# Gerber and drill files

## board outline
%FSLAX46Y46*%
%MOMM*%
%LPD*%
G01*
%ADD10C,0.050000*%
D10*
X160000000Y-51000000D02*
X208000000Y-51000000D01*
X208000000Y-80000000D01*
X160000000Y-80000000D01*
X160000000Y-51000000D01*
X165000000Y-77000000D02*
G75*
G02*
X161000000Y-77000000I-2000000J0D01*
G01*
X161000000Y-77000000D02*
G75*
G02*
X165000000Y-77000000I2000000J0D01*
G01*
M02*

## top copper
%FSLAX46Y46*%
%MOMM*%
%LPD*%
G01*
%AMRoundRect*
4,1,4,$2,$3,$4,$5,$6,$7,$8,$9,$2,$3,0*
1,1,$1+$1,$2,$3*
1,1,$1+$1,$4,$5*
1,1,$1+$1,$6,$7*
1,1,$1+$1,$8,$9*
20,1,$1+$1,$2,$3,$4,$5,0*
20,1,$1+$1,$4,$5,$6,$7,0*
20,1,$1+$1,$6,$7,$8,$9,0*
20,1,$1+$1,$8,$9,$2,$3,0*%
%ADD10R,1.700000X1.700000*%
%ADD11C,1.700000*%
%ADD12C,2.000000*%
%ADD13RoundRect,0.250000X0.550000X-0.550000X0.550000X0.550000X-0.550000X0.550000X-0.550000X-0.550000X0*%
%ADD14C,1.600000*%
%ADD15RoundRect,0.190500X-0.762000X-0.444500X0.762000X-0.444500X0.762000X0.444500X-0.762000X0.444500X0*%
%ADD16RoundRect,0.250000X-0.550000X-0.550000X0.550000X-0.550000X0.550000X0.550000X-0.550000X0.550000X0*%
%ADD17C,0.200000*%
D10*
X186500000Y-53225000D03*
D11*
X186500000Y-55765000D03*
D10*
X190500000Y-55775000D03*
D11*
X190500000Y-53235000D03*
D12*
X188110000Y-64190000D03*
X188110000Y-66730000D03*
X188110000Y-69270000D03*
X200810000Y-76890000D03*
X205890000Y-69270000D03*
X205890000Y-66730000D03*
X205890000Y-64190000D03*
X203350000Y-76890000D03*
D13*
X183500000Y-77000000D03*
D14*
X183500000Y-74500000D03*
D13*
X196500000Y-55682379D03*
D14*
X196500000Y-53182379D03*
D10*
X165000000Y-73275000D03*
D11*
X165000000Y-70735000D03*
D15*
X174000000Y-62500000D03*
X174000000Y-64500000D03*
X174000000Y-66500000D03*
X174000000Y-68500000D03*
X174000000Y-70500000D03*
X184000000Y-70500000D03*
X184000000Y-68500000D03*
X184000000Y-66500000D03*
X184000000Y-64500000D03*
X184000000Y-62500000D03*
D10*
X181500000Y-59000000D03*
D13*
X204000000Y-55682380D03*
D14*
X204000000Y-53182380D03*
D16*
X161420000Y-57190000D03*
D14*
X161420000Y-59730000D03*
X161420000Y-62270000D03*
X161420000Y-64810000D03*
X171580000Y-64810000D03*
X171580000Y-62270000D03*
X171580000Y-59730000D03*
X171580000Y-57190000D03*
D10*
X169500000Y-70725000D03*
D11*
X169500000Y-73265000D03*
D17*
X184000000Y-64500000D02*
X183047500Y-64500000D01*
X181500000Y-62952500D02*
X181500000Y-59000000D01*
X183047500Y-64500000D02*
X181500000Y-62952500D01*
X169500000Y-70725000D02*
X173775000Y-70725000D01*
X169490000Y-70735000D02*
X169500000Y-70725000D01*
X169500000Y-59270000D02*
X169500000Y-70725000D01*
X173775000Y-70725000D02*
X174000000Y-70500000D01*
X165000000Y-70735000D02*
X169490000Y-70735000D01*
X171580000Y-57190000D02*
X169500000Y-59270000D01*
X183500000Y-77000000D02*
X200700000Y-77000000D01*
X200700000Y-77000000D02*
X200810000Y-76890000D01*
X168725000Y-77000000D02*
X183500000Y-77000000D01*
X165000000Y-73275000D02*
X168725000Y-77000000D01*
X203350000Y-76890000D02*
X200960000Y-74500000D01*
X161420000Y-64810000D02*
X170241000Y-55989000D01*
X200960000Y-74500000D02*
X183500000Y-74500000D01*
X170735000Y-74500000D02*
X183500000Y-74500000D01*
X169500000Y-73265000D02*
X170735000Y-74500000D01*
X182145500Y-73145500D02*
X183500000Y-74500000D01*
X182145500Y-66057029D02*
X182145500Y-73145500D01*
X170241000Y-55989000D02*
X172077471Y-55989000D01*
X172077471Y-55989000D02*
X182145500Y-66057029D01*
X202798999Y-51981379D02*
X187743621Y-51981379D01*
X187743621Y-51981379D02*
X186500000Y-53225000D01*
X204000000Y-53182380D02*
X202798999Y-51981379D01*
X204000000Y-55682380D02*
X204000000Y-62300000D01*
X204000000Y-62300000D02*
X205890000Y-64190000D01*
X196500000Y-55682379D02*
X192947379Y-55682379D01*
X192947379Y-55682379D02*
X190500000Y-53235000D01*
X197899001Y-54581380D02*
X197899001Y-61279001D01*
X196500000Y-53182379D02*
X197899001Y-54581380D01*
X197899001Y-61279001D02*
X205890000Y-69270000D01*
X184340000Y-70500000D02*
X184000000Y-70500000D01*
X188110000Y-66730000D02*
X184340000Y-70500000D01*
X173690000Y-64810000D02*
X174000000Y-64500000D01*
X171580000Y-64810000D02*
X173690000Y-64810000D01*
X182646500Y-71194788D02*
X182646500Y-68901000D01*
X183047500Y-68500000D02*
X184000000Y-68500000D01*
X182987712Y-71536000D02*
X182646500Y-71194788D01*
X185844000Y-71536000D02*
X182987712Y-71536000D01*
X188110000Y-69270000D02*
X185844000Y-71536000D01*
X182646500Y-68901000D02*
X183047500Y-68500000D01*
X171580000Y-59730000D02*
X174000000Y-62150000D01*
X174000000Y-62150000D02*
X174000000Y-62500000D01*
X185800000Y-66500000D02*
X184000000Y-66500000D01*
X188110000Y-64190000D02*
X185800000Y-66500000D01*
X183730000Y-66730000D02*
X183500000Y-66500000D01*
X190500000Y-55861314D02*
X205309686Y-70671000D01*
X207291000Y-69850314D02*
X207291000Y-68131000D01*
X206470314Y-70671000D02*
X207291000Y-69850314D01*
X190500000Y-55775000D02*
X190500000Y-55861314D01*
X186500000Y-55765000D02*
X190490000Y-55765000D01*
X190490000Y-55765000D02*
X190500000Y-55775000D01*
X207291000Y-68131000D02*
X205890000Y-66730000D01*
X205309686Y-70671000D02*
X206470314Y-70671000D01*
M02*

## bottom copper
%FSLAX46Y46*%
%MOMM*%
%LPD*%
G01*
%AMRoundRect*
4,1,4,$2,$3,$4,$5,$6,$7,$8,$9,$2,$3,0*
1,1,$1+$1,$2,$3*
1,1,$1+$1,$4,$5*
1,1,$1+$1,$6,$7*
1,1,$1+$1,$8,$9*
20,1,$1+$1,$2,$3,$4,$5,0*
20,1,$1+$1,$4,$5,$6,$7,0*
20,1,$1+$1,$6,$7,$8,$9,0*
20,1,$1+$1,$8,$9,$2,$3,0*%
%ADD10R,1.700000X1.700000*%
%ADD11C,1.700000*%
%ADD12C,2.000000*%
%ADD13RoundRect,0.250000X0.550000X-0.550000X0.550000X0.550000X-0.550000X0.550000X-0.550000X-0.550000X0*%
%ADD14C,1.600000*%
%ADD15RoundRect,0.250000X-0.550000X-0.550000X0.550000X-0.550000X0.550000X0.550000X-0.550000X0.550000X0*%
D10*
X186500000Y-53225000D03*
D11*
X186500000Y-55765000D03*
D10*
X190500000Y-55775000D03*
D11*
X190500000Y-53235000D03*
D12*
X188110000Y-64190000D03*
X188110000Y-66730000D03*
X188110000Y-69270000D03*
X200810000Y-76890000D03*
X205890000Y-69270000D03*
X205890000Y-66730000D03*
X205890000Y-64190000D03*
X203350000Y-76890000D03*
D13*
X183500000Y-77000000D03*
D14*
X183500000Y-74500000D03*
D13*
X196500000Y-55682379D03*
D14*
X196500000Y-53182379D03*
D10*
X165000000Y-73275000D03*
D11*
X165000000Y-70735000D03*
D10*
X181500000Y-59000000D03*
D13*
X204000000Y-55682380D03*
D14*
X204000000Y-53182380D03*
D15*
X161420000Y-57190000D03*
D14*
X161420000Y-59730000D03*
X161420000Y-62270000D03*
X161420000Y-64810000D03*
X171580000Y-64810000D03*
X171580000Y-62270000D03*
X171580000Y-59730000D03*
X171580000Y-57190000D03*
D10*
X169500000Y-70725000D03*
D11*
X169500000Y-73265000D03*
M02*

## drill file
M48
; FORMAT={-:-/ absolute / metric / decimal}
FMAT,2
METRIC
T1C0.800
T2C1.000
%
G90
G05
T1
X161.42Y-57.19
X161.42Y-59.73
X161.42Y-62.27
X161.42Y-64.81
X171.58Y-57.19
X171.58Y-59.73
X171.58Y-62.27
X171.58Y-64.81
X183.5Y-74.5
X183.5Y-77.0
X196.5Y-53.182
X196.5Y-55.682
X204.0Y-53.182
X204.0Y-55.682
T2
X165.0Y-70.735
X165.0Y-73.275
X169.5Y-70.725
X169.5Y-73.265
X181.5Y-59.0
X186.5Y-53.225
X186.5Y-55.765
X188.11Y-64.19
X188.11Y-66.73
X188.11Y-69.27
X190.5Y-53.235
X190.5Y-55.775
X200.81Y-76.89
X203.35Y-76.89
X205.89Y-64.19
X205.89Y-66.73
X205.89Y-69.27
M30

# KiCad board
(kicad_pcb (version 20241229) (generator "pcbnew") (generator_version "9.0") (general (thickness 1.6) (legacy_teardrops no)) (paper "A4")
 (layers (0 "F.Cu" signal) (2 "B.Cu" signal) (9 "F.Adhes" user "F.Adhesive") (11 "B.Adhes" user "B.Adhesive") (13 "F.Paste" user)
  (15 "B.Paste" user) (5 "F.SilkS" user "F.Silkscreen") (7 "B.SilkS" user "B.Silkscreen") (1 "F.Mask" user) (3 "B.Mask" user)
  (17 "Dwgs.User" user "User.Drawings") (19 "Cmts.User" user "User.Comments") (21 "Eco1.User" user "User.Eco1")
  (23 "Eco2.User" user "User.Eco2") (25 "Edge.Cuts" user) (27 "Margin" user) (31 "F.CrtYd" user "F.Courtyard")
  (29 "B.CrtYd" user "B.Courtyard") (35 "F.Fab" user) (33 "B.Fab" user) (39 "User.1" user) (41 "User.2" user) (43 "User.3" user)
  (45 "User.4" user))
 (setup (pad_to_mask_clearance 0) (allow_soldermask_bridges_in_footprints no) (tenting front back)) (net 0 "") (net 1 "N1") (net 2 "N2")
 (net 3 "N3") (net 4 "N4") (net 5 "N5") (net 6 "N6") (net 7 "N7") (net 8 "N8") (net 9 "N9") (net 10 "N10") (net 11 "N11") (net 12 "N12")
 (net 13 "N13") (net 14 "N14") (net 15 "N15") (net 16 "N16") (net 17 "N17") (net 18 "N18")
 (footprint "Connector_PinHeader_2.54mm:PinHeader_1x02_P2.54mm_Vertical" (layer "F.Cu") (at 186.5 53.225)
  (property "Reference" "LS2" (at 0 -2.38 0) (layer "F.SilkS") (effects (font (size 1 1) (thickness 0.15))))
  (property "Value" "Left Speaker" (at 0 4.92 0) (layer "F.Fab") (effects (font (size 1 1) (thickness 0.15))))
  (pad "1" thru_hole rect (at 0 0) (size 1.7 1.7) (drill 1) (layers "*.Cu" "*.Mask") (remove_unused_layers no) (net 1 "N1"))
  (pad "2" thru_hole circle (at 0 2.54) (size 1.7 1.7) (drill 1) (layers "*.Cu" "*.Mask") (remove_unused_layers no) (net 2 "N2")))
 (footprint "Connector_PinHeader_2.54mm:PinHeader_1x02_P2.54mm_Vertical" (layer "F.Cu") (at 190.5 55.775 180)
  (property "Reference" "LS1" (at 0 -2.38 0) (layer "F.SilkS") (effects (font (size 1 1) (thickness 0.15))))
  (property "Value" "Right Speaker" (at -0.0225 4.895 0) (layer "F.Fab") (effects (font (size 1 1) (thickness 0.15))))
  (pad "1" thru_hole rect (at 0 0 180) (size 1.7 1.7) (drill 1) (layers "*.Cu" "*.Mask") (remove_unused_layers no) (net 2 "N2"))
  (pad "2" thru_hole circle (at 0 2.54 180) (size 1.7 1.7) (drill 1) (layers "*.Cu" "*.Mask") (remove_unused_layers no) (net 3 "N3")))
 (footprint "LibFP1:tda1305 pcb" (layer "F.Cu") (at 198.27 66.73)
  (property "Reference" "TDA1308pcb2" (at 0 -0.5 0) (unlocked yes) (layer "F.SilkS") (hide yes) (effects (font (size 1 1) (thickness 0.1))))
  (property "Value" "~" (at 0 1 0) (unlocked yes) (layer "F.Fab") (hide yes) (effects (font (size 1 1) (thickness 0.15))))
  (pad "1" thru_hole circle (at -10.16 -2.54) (size 2 2) (drill 1) (layers "*.Cu" "*.Mask") (remove_unused_layers no) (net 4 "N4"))
  (pad "2" thru_hole circle (at -10.16 0) (size 2 2) (drill 1) (layers "*.Cu" "*.Mask") (remove_unused_layers no) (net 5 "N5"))
  (pad "3" thru_hole circle (at -10.16 2.54) (size 2 2) (drill 1) (layers "*.Cu" "*.Mask") (remove_unused_layers no) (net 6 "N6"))
  (pad "4" thru_hole circle (at 2.54 10.16) (size 2 2) (drill 1) (layers "*.Cu" "*.Mask") (remove_unused_layers no) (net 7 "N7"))
  (pad "5" thru_hole circle (at 7.62 2.54) (size 2 2) (drill 1) (layers "*.Cu" "*.Mask") (remove_unused_layers no) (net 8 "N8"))
  (pad "6" thru_hole circle (at 7.62 0) (size 2 2) (drill 1) (layers "*.Cu" "*.Mask") (remove_unused_layers no) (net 2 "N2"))
  (pad "7" thru_hole circle (at 7.62 -2.54) (size 2 2) (drill 1) (layers "*.Cu" "*.Mask") (remove_unused_layers no) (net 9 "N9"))
  (pad "8" thru_hole circle (at 5.08 10.16) (size 2 2) (drill 1) (layers "*.Cu" "*.Mask") (remove_unused_layers no) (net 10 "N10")))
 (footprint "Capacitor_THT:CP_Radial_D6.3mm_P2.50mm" (layer "F.Cu") (at 183.5 77 90)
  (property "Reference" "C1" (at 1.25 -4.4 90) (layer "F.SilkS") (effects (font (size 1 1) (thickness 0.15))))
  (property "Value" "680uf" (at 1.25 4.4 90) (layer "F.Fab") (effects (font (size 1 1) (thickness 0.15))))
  (pad "1" thru_hole roundrect (at 0 0 90) (size 1.6 1.6) (drill 0.8) (layers "*.Cu" "*.Mask") (remove_unused_layers no)
   (roundrect_rratio 0.15625) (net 7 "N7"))
  (pad "2" thru_hole circle (at 2.5 0 90) (size 1.6 1.6) (drill 0.8) (layers "*.Cu" "*.Mask") (remove_unused_layers no) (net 10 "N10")))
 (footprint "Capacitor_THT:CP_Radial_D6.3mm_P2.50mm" (layer "F.Cu") (at 196.5 55.682379 90)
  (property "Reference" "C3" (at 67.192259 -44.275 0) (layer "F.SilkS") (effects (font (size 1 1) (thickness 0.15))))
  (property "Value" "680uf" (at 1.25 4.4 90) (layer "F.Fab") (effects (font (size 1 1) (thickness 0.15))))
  (pad "1" thru_hole roundrect (at 0 0 90) (size 1.6 1.6) (drill 0.8) (layers "*.Cu" "*.Mask") (remove_unused_layers no)
   (roundrect_rratio 0.15625) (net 3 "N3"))
  (pad "2" thru_hole circle (at 2.5 0 90) (size 1.6 1.6) (drill 0.8) (layers "*.Cu" "*.Mask") (remove_unused_layers no) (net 8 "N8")))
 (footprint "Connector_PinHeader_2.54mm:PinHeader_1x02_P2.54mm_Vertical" (layer "F.Cu") (at 165 73.275 180)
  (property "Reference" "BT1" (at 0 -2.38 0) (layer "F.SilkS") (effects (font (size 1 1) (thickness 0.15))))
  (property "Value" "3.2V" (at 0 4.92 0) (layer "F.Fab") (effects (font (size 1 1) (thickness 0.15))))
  (pad "1" thru_hole rect (at 0 0 180) (size 1.7 1.7) (drill 1) (layers "*.Cu" "*.Mask") (remove_unused_layers no) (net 7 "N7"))
  (pad "2" thru_hole circle (at 0 2.54 180) (size 1.7 1.7) (drill 1) (layers "*.Cu" "*.Mask") (remove_unused_layers no) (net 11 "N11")))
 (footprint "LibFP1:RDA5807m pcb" (layer "F.Cu") (at 179 66.5)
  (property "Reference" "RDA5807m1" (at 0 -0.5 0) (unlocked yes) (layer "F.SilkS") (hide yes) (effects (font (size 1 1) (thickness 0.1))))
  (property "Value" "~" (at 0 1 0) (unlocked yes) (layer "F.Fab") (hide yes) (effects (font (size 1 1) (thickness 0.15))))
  (pad "1" smd roundrect (at -5 -4) (size 1.905 1.27) (layers "F.Cu" "F.Mask" "F.Paste") (roundrect_rratio 0.15) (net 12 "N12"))
  (pad "2" smd roundrect (at -5 -2) (size 1.905 1.27) (layers "F.Cu" "F.Mask" "F.Paste") (roundrect_rratio 0.15) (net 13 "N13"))
  (pad "3" smd roundrect (at -5 0) (size 1.905 1.27) (layers "F.Cu" "F.Mask" "F.Paste") (roundrect_rratio 0.15))
  (pad "4" smd roundrect (at -5 2) (size 1.905 1.27) (layers "F.Cu" "F.Mask" "F.Paste") (roundrect_rratio 0.15))
  (pad "5" smd roundrect (at -5 4) (size 1.905 1.27) (layers "F.Cu" "F.Mask" "F.Paste") (roundrect_rratio 0.15) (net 11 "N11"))
  (pad "6" smd roundrect (at 5 4) (size 1.905 1.27) (layers "F.Cu" "F.Mask" "F.Paste") (roundrect_rratio 0.15) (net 5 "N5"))
  (pad "7" smd roundrect (at 5 2) (size 1.905 1.27) (layers "F.Cu" "F.Mask" "F.Paste") (roundrect_rratio 0.15) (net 6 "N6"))
  (pad "8" smd roundrect (at 5 0) (size 1.905 1.27) (layers "F.Cu" "F.Mask" "F.Paste") (roundrect_rratio 0.15) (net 4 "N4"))
  (pad "9" smd roundrect (at 5 -2) (size 1.905 1.27) (layers "F.Cu" "F.Mask" "F.Paste") (roundrect_rratio 0.15) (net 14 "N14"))
  (pad "10" smd roundrect (at 5 -4) (size 1.905 1.27) (layers "F.Cu" "F.Mask" "F.Paste") (roundrect_rratio 0.15)))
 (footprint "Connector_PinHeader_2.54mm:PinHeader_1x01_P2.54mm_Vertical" (layer "F.Cu") (at 181.5 59)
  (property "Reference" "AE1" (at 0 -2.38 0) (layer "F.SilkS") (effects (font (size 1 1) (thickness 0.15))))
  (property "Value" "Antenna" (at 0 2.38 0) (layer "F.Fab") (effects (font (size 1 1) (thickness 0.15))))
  (pad "1" thru_hole rect (at 0 0) (size 1.7 1.7) (drill 1) (layers "*.Cu" "*.Mask") (remove_unused_layers no) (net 14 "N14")))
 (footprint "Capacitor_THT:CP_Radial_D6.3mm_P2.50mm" (layer "F.Cu") (at 204 55.68238 90)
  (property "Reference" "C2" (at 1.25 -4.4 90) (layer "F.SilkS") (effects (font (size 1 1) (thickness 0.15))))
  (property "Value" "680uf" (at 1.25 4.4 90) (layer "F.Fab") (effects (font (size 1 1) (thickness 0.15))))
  (pad "1" thru_hole roundrect (at 0 0 90) (size 1.6 1.6) (drill 0.8) (layers "*.Cu" "*.Mask") (remove_unused_layers no)
   (roundrect_rratio 0.15625) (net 9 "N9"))
  (pad "2" thru_hole circle (at 2.5 0 90) (size 1.6 1.6) (drill 0.8) (layers "*.Cu" "*.Mask") (remove_unused_layers no) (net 1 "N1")))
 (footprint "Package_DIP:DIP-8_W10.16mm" (layer "F.Cu") (at 161.42 57.19)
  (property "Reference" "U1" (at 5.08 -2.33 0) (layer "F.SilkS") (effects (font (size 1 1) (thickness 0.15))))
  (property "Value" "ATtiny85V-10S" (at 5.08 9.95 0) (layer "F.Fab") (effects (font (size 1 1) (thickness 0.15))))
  (pad "1" thru_hole roundrect (at 0 0) (size 1.6 1.6) (drill 0.8) (layers "*.Cu" "*.Mask") (remove_unused_layers no)
   (roundrect_rratio 0.15625) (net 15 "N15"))
  (pad "2" thru_hole circle (at 0 2.54) (size 1.6 1.6) (drill 0.8) (layers "*.Cu" "*.Mask") (remove_unused_layers no) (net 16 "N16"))
  (pad "3" thru_hole circle (at 0 5.08) (size 1.6 1.6) (drill 0.8) (layers "*.Cu" "*.Mask") (remove_unused_layers no) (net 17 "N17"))
  (pad "4" thru_hole circle (at 0 7.62) (size 1.6 1.6) (drill 0.8) (layers "*.Cu" "*.Mask") (remove_unused_layers no) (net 10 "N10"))
  (pad "5" thru_hole circle (at 10.16 7.62) (size 1.6 1.6) (drill 0.8) (layers "*.Cu" "*.Mask") (remove_unused_layers no) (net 13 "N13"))
  (pad "6" thru_hole circle (at 10.16 5.08) (size 1.6 1.6) (drill 0.8) (layers "*.Cu" "*.Mask") (remove_unused_layers no) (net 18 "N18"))
  (pad "7" thru_hole circle (at 10.16 2.54) (size 1.6 1.6) (drill 0.8) (layers "*.Cu" "*.Mask") (remove_unused_layers no) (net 12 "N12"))
  (pad "8" thru_hole circle (at 10.16 0) (size 1.6 1.6) (drill 0.8) (layers "*.Cu" "*.Mask") (remove_unused_layers no) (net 11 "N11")))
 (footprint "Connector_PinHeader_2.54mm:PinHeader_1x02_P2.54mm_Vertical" (layer "F.Cu") (at 169.5 70.725)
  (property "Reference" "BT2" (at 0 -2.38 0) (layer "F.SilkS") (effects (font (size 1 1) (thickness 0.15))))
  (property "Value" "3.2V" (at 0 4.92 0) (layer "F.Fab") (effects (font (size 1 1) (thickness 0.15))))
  (pad "1" thru_hole rect (at 0 0) (size 1.7 1.7) (drill 1) (layers "*.Cu" "*.Mask") (remove_unused_layers no) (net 11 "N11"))
  (pad "2" thru_hole circle (at 0 2.54) (size 1.7 1.7) (drill 1) (layers "*.Cu" "*.Mask") (remove_unused_layers no) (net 10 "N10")))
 (gr_rect (start 160 51) (end 208 80) (stroke (width 0.05) (type default)) (fill no) (layer "Edge.Cuts"))
 (gr_circle (center 163 77) (end 163 79) (stroke (width 0.05) (type default)) (fill no) (layer "Edge.Cuts"))
 (segment (start 184 64.5) (end 183.0475 64.5) (width 0.2) (layer "F.Cu") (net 14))
 (segment (start 181.5 62.9525) (end 181.5 59) (width 0.2) (layer "F.Cu") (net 14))
 (segment (start 183.0475 64.5) (end 181.5 62.9525) (width 0.2) (layer "F.Cu") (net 14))
 (segment (start 169.5 70.725) (end 173.775 70.725) (width 0.2) (layer "F.Cu") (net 11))
 (segment (start 169.49 70.735) (end 169.5 70.725) (width 0.2) (layer "F.Cu") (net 11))
 (segment (start 169.5 59.27) (end 169.5 70.725) (width 0.2) (layer "F.Cu") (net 11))
 (segment (start 173.775 70.725) (end 174 70.5) (width 0.2) (layer "F.Cu") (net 11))
 (segment (start 165 70.735) (end 169.49 70.735) (width 0.2) (layer "F.Cu") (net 11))
 (segment (start 171.58 57.19) (end 169.5 59.27) (width 0.2) (layer "F.Cu") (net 11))
 (segment (start 183.5 77) (end 200.7 77) (width 0.2) (layer "F.Cu") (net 7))
 (segment (start 200.7 77) (end 200.81 76.89) (width 0.2) (layer "F.Cu") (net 7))
 (segment (start 168.725 77) (end 183.5 77) (width 0.2) (layer "F.Cu") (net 7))
 (segment (start 165 73.275) (end 168.725 77) (width 0.2) (layer "F.Cu") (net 7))
 (segment (start 203.35 76.89) (end 200.96 74.5) (width 0.2) (layer "F.Cu") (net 10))
 (segment (start 161.42 64.81) (end 170.241 55.989) (width 0.2) (layer "F.Cu") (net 10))
 (segment (start 200.96 74.5) (end 183.5 74.5) (width 0.2) (layer "F.Cu") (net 10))
 (segment (start 170.735 74.5) (end 183.5 74.5) (width 0.2) (layer "F.Cu") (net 10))
 (segment (start 169.5 73.265) (end 170.735 74.5) (width 0.2) (layer "F.Cu") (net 10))
 (segment (start 182.1455 73.1455) (end 183.5 74.5) (width 0.2) (layer "F.Cu") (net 10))
 (segment (start 182.1455 66.057029) (end 182.1455 73.1455) (width 0.2) (layer "F.Cu") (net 10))
 (segment (start 170.241 55.989) (end 172.077471 55.989) (width 0.2) (layer "F.Cu") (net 10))
 (segment (start 172.077471 55.989) (end 182.1455 66.057029) (width 0.2) (layer "F.Cu") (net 10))
 (segment (start 202.798999 51.981379) (end 187.743621 51.981379) (width 0.2) (layer "F.Cu") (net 1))
 (segment (start 187.743621 51.981379) (end 186.5 53.225) (width 0.2) (layer "F.Cu") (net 1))
 (segment (start 204 53.18238) (end 202.798999 51.981379) (width 0.2) (layer "F.Cu") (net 1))
 (segment (start 204 55.68238) (end 204 62.3) (width 0.2) (layer "F.Cu") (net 9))
 (segment (start 204 62.3) (end 205.89 64.19) (width 0.2) (layer "F.Cu") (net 9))
 (segment (start 196.5 55.682379) (end 192.947379 55.682379) (width 0.2) (layer "F.Cu") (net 3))
 (segment (start 192.947379 55.682379) (end 190.5 53.235) (width 0.2) (layer "F.Cu") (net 3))
 (segment (start 197.899001 54.58138) (end 197.899001 61.279001) (width 0.2) (layer "F.Cu") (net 8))
 (segment (start 196.5 53.182379) (end 197.899001 54.58138) (width 0.2) (layer "F.Cu") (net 8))
 (segment (start 197.899001 61.279001) (end 205.89 69.27) (width 0.2) (layer "F.Cu") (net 8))
 (segment (start 184.34 70.5) (end 184 70.5) (width 0.2) (layer "F.Cu") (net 5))
 (segment (start 188.11 66.73) (end 184.34 70.5) (width 0.2) (layer "F.Cu") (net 5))
 (segment (start 173.69 64.81) (end 174 64.5) (width 0.2) (layer "F.Cu") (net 13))
 (segment (start 171.58 64.81) (end 173.69 64.81) (width 0.2) (layer "F.Cu") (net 13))
 (segment (start 182.6465 71.194788) (end 182.6465 68.901) (width 0.2) (layer "F.Cu") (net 6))
 (segment (start 183.0475 68.5) (end 184 68.5) (width 0.2) (layer "F.Cu") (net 6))
 (segment (start 182.987712 71.536) (end 182.6465 71.194788) (width 0.2) (layer "F.Cu") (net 6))
 (segment (start 185.844 71.536) (end 182.987712 71.536) (width 0.2) (layer "F.Cu") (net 6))
 (segment (start 188.11 69.27) (end 185.844 71.536) (width 0.2) (layer "F.Cu") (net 6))
 (segment (start 182.6465 68.901) (end 183.0475 68.5) (width 0.2) (layer "F.Cu") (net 6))
 (segment (start 171.58 59.73) (end 174 62.15) (width 0.2) (layer "F.Cu") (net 12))
 (segment (start 174 62.15) (end 174 62.5) (width 0.2) (layer "F.Cu") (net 12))
 (segment (start 185.8 66.5) (end 184 66.5) (width 0.2) (layer "F.Cu") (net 4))
 (segment (start 188.11 64.19) (end 185.8 66.5) (width 0.2) (layer "F.Cu") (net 4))
 (segment (start 183.73 66.73) (end 183.5 66.5) (width 0.2) (layer "F.Cu") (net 4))
 (segment (start 190.5 55.861314) (end 205.309686 70.671) (width 0.2) (layer "F.Cu") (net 2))
 (segment (start 207.291 69.850314) (end 207.291 68.131) (width 0.2) (layer "F.Cu") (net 2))
 (segment (start 206.470314 70.671) (end 207.291 69.850314) (width 0.2) (layer "F.Cu") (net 2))
 (segment (start 190.5 55.775) (end 190.5 55.861314) (width 0.2) (layer "F.Cu") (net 2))
 (segment (start 186.5 55.765) (end 190.49 55.765) (width 0.2) (layer "F.Cu") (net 2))
 (segment (start 190.49 55.765) (end 190.5 55.775) (width 0.2) (layer "F.Cu") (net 2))
 (segment (start 207.291 68.131) (end 205.89 66.73) (width 0.2) (layer "F.Cu") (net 2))
 (segment (start 205.309686 70.671) (end 206.470314 70.671) (width 0.2) (layer "F.Cu") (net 2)))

